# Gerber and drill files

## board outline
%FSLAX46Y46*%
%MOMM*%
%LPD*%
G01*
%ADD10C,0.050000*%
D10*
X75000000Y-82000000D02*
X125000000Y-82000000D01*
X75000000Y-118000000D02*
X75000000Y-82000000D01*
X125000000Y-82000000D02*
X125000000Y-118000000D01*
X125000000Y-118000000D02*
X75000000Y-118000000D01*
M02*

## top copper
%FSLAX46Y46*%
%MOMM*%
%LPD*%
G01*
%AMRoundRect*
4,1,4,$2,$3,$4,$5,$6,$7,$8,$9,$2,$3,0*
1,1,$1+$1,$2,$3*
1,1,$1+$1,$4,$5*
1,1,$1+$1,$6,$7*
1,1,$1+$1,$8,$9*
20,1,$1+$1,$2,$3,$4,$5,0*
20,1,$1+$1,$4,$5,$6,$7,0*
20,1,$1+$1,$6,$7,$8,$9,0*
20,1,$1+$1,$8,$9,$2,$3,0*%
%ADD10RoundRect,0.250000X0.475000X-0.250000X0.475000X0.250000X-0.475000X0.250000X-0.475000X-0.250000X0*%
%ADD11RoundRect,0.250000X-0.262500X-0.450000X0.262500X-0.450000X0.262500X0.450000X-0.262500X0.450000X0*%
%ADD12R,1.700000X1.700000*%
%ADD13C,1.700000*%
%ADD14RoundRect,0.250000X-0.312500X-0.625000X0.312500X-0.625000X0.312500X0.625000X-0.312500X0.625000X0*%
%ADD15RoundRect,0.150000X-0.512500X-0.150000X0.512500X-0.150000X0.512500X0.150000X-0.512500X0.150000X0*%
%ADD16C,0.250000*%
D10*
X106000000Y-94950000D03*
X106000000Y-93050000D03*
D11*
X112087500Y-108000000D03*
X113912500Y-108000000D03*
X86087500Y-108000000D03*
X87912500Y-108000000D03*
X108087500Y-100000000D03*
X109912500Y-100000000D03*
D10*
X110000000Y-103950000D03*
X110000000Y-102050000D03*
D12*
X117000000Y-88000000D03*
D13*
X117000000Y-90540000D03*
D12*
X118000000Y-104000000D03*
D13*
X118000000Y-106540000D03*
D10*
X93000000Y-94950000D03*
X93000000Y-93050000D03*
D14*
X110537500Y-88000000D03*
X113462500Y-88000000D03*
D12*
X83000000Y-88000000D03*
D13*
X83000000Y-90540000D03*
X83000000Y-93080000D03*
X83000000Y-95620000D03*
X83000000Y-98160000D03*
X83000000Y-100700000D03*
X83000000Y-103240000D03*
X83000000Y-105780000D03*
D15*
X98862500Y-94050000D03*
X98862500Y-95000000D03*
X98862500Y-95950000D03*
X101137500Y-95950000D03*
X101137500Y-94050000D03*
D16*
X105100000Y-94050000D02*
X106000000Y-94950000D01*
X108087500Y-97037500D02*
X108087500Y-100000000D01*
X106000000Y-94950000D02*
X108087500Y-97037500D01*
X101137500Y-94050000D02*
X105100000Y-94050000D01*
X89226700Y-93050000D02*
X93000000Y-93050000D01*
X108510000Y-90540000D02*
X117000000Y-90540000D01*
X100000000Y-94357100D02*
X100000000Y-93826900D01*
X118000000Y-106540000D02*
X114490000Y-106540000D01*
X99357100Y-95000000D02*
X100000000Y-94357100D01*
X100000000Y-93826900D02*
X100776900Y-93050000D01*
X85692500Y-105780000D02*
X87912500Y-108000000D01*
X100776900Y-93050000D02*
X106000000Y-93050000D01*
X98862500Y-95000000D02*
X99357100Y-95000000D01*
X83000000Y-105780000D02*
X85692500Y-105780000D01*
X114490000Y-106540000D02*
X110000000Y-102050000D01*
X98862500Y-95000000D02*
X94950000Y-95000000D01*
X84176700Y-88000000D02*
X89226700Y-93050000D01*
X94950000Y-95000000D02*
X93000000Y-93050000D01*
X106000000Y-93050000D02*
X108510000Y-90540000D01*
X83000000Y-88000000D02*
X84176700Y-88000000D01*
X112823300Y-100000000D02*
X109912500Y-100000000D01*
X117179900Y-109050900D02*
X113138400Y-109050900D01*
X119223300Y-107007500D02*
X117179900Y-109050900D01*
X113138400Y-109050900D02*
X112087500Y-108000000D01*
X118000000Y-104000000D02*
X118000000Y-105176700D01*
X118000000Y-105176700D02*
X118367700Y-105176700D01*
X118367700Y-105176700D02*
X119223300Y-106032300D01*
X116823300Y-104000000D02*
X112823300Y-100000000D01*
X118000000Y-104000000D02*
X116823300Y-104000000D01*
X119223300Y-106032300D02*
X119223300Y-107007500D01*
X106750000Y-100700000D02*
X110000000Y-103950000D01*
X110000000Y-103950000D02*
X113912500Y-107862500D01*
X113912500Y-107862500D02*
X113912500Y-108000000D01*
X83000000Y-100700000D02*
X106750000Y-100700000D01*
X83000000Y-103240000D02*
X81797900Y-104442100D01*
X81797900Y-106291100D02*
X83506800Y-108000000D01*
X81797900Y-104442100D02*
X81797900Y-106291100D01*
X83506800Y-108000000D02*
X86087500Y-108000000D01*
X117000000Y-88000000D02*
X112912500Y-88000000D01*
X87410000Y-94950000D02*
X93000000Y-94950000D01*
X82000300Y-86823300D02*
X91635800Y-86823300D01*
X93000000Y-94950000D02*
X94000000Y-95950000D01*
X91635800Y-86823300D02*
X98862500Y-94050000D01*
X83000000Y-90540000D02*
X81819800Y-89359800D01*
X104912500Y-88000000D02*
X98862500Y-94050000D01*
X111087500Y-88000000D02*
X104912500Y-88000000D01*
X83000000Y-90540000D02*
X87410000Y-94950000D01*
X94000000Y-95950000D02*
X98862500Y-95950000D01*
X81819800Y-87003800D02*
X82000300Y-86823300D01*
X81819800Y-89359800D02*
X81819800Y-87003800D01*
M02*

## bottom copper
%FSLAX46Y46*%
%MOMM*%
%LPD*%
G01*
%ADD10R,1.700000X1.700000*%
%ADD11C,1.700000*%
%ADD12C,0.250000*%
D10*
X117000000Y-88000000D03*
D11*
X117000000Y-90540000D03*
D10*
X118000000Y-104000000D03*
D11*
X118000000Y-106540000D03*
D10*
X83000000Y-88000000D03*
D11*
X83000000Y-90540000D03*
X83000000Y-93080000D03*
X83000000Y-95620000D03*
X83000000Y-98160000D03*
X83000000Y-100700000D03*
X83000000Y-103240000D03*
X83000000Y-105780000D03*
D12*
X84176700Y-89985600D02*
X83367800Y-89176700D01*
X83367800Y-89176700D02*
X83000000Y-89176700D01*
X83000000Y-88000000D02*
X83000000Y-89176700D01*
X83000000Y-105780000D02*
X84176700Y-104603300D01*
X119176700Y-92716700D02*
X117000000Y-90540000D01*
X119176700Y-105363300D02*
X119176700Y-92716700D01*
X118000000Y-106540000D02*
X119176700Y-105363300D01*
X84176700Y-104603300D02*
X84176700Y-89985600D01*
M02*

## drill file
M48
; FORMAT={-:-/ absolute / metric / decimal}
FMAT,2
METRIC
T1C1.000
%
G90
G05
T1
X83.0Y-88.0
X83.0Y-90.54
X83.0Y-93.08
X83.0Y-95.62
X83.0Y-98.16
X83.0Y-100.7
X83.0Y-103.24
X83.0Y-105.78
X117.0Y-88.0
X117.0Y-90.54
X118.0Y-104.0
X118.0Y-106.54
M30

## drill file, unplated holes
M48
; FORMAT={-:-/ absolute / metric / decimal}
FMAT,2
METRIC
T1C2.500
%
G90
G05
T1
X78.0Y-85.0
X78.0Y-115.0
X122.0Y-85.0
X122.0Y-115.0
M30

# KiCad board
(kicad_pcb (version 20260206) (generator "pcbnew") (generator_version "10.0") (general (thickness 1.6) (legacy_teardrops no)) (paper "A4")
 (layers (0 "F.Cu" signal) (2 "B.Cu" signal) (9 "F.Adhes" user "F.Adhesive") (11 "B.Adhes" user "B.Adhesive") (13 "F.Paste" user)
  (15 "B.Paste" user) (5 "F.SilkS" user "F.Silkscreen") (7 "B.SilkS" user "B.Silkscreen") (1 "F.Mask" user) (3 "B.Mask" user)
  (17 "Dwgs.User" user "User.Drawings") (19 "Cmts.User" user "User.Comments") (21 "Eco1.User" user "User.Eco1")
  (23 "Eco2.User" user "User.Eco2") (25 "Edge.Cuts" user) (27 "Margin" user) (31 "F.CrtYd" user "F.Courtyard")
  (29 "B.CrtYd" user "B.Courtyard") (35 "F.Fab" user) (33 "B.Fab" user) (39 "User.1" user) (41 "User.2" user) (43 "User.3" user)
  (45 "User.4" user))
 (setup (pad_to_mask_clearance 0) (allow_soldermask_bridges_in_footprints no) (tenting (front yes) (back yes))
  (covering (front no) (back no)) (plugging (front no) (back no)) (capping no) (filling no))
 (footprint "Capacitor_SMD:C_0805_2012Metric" (layer "F.Cu") (at 106 94 90)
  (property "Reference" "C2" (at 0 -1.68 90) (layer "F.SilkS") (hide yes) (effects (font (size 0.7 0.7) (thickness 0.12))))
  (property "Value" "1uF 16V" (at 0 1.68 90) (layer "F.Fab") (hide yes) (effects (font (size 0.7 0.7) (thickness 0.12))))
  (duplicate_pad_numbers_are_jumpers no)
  (pad "1" smd roundrect (at -0.95 0 90) (size 1 1.45) (layers "F.Cu" "F.Mask" "F.Paste") (roundrect_rratio 0.25) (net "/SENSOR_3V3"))
  (pad "2" smd roundrect (at 0.95 0 90) (size 1 1.45) (layers "F.Cu" "F.Mask" "F.Paste") (roundrect_rratio 0.25) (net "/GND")))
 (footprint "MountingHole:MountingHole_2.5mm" (layer "F.Cu") (at 78 85)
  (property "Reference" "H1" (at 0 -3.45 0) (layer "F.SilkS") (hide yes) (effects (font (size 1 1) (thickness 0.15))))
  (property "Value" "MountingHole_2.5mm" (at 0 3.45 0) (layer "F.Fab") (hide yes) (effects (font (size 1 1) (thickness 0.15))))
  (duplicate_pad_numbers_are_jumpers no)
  (pad "" np_thru_hole circle (at 0 0) (size 2.5 2.5) (drill 2.5) (layers "*.Cu" "*.Mask")))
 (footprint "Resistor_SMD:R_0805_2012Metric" (layer "F.Cu") (at 113 108)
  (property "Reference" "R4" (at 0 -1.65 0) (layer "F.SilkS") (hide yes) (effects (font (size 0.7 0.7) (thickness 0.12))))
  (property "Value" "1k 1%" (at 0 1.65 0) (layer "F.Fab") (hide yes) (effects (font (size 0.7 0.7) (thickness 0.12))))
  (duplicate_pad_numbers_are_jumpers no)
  (pad "1" smd roundrect (at -0.9125 0) (size 1.025 1.4) (layers "F.Cu" "F.Mask" "F.Paste") (roundrect_rratio 0.243902) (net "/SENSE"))
  (pad "2" smd roundrect (at 0.9125 0) (size 1.025 1.4) (layers "F.Cu" "F.Mask" "F.Paste") (roundrect_rratio 0.243902) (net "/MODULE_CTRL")))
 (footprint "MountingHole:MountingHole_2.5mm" (layer "F.Cu") (at 122 85)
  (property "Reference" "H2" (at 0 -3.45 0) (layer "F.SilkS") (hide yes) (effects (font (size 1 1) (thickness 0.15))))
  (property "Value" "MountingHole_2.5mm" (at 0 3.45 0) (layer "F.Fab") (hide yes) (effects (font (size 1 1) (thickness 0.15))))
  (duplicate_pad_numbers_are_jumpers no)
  (pad "" np_thru_hole circle (at 0 0) (size 2.5 2.5) (drill 2.5) (layers "*.Cu" "*.Mask")))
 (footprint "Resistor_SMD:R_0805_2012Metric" (layer "F.Cu") (at 87 108)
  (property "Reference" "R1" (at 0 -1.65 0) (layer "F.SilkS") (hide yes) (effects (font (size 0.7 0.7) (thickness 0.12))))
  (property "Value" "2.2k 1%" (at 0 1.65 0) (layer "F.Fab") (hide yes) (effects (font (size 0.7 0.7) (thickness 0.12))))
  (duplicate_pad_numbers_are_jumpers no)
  (pad "1" smd roundrect (at -0.9125 0) (size 1.025 1.4) (layers "F.Cu" "F.Mask" "F.Paste") (roundrect_rratio 0.243902) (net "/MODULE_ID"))
  (pad "2" smd roundrect (at 0.9125 0) (size 1.025 1.4) (layers "F.Cu" "F.Mask" "F.Paste") (roundrect_rratio 0.243902) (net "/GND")))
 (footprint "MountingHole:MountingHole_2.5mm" (layer "F.Cu") (at 78 115)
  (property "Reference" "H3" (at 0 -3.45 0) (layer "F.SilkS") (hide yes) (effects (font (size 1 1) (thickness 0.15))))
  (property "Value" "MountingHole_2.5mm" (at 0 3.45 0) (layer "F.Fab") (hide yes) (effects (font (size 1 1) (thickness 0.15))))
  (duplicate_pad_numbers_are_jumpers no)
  (pad "" np_thru_hole circle (at 0 0) (size 2.5 2.5) (drill 2.5) (layers "*.Cu" "*.Mask")))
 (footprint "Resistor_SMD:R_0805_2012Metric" (layer "F.Cu") (at 109 100)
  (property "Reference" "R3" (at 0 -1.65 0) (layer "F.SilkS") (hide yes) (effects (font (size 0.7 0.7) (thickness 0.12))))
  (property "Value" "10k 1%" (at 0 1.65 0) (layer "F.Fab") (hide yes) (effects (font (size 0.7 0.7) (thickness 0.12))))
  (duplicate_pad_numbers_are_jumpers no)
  (pad "1" smd roundrect (at -0.9125 0) (size 1.025 1.4) (layers "F.Cu" "F.Mask" "F.Paste") (roundrect_rratio 0.243902) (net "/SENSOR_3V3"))
  (pad "2" smd roundrect (at 0.9125 0) (size 1.025 1.4) (layers "F.Cu" "F.Mask" "F.Paste") (roundrect_rratio 0.243902) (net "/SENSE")))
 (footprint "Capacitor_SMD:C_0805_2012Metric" (layer "F.Cu") (at 110 103 90)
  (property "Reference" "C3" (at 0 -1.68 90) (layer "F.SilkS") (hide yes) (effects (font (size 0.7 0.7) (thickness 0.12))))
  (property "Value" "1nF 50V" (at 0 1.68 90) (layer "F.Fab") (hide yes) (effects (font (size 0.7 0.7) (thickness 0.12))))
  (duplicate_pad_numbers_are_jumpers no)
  (pad "1" smd roundrect (at -0.95 0 90) (size 1 1.45) (layers "F.Cu" "F.Mask" "F.Paste") (roundrect_rratio 0.25) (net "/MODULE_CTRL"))
  (pad "2" smd roundrect (at 0.95 0 90) (size 1 1.45) (layers "F.Cu" "F.Mask" "F.Paste") (roundrect_rratio 0.25) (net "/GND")))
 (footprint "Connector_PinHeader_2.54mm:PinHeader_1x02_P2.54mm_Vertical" (layer "F.Cu") (at 117 88)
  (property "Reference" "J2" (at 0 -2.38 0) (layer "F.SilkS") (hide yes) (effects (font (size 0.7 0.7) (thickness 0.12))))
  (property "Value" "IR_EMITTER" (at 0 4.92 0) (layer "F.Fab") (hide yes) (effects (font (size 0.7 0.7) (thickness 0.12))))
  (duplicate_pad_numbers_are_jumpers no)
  (pad "1" thru_hole rect (at 0 0) (size 1.7 1.7) (drill 1) (layers "*.Cu" "*.Mask") (remove_unused_layers no) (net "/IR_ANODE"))
  (pad "2" thru_hole circle (at 0 2.54) (size 1.7 1.7) (drill 1) (layers "*.Cu" "*.Mask") (remove_unused_layers no) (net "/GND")))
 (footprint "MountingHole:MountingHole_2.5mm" (layer "F.Cu") (at 122 115)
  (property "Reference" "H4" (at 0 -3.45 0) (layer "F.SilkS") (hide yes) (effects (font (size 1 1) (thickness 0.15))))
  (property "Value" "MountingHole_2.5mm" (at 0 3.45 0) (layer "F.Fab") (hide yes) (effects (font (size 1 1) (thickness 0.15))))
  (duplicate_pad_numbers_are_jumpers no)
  (pad "" np_thru_hole circle (at 0 0) (size 2.5 2.5) (drill 2.5) (layers "*.Cu" "*.Mask")))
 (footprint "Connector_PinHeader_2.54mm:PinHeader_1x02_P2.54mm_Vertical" (layer "F.Cu") (at 118 104)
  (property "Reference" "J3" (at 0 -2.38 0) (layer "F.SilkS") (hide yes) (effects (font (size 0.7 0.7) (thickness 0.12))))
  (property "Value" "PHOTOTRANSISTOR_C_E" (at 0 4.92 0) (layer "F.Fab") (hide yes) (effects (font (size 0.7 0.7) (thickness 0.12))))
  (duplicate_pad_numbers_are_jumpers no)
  (pad "1" thru_hole rect (at 0 0) (size 1.7 1.7) (drill 1) (layers "*.Cu" "*.Mask") (remove_unused_layers no) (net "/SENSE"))
  (pad "2" thru_hole circle (at 0 2.54) (size 1.7 1.7) (drill 1) (layers "*.Cu" "*.Mask") (remove_unused_layers no) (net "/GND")))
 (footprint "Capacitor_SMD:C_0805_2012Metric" (layer "F.Cu") (at 93 94 90)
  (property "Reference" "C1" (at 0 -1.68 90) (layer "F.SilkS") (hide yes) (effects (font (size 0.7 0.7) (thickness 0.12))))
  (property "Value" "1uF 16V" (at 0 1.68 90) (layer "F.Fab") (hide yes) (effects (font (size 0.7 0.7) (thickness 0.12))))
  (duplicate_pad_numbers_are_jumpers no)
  (pad "1" smd roundrect (at -0.95 0 90) (size 1 1.45) (layers "F.Cu" "F.Mask" "F.Paste") (roundrect_rratio 0.25) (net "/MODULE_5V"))
  (pad "2" smd roundrect (at 0.95 0 90) (size 1 1.45) (layers "F.Cu" "F.Mask" "F.Paste") (roundrect_rratio 0.25) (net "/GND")))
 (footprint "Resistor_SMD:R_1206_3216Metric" (layer "F.Cu") (at 112 88)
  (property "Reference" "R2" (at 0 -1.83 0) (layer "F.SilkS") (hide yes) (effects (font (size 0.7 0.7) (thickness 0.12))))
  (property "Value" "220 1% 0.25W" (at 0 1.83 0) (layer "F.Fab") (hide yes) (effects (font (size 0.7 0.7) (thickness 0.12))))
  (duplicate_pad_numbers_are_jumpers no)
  (pad "1" smd roundrect (at -1.4625 0) (size 1.125 1.75) (layers "F.Cu" "F.Mask" "F.Paste") (roundrect_rratio 0.222222) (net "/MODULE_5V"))
  (pad "2" smd roundrect (at 1.4625 0) (size 1.125 1.75) (layers "F.Cu" "F.Mask" "F.Paste") (roundrect_rratio 0.222222) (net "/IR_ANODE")))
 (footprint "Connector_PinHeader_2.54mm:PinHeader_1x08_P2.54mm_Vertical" (layer "F.Cu") (at 83 88)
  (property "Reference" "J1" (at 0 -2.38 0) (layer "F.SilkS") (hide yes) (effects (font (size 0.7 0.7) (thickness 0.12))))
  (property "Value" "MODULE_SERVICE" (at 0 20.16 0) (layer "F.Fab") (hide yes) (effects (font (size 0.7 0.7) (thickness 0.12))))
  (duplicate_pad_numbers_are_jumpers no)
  (pad "1" thru_hole rect (at 0 0) (size 1.7 1.7) (drill 1) (layers "*.Cu" "*.Mask") (remove_unused_layers no) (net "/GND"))
  (pad "2" thru_hole circle (at 0 2.54) (size 1.7 1.7) (drill 1) (layers "*.Cu" "*.Mask") (remove_unused_layers no) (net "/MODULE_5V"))
  (pad "3" thru_hole circle (at 0 5.08) (size 1.7 1.7) (drill 1) (layers "*.Cu" "*.Mask") (remove_unused_layers no)
   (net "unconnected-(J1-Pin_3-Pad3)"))
  (pad "4" thru_hole circle (at 0 7.62) (size 1.7 1.7) (drill 1) (layers "*.Cu" "*.Mask") (remove_unused_layers no)
   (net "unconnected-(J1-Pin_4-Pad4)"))
  (pad "5" thru_hole circle (at 0 10.16) (size 1.7 1.7) (drill 1) (layers "*.Cu" "*.Mask") (remove_unused_layers no)
   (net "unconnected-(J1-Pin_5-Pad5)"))
  (pad "6" thru_hole circle (at 0 12.7) (size 1.7 1.7) (drill 1) (layers "*.Cu" "*.Mask") (remove_unused_layers no) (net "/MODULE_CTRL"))
  (pad "7" thru_hole circle (at 0 15.24) (size 1.7 1.7) (drill 1) (layers "*.Cu" "*.Mask") (remove_unused_layers no) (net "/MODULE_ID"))
  (pad "8" thru_hole circle (at 0 17.78) (size 1.7 1.7) (drill 1) (layers "*.Cu" "*.Mask") (remove_unused_layers no) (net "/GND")))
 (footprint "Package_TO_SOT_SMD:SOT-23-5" (layer "F.Cu") (at 100 95)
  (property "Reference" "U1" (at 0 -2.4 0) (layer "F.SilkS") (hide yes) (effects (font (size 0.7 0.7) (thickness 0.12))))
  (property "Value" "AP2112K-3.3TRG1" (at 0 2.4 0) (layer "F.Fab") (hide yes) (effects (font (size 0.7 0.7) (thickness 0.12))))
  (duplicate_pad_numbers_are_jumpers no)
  (pad "1" smd roundrect (at -1.1375 -0.95) (size 1.325 0.6) (layers "F.Cu" "F.Mask" "F.Paste") (roundrect_rratio 0.25) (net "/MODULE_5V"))
  (pad "2" smd roundrect (at -1.1375 0) (size 1.325 0.6) (layers "F.Cu" "F.Mask" "F.Paste") (roundrect_rratio 0.25) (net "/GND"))
  (pad "3" smd roundrect (at -1.1375 0.95) (size 1.325 0.6) (layers "F.Cu" "F.Mask" "F.Paste") (roundrect_rratio 0.25) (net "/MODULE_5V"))
  (pad "4" smd roundrect (at 1.1375 0.95) (size 1.325 0.6) (layers "F.Cu" "F.Mask" "F.Paste") (roundrect_rratio 0.25)
   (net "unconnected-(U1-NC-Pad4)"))
  (pad "5" smd roundrect (at 1.1375 -0.95) (size 1.325 0.6) (layers "F.Cu" "F.Mask" "F.Paste") (roundrect_rratio 0.25) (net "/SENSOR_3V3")))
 (gr_line (start 75 82) (end 125 82) (stroke (width 0.05) (type default)) (layer "Edge.Cuts"))
 (gr_line (start 75 118) (end 75 82) (stroke (width 0.05) (type default)) (layer "Edge.Cuts"))
 (gr_line (start 125 82) (end 125 118) (stroke (width 0.05) (type default)) (layer "Edge.Cuts"))
 (gr_line (start 125 118) (end 75 118) (stroke (width 0.05) (type default)) (layer "Edge.Cuts"))
 (segment (start 105.1 94.05) (end 106 94.95) (width 0.25) (layer "F.Cu") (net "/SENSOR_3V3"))
 (segment (start 108.0875 97.0375) (end 108.0875 100) (width 0.25) (layer "F.Cu") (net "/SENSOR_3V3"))
 (segment (start 106 94.95) (end 108.0875 97.0375) (width 0.25) (layer "F.Cu") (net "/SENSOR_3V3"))
 (segment (start 101.1375 94.05) (end 105.1 94.05) (width 0.25) (layer "F.Cu") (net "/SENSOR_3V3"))
 (segment (start 89.2267 93.05) (end 93 93.05) (width 0.25) (layer "F.Cu") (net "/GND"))
 (segment (start 108.51 90.54) (end 117 90.54) (width 0.25) (layer "F.Cu") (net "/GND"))
 (segment (start 100 94.3571) (end 100 93.8269) (width 0.25) (layer "F.Cu") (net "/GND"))
 (segment (start 118 106.54) (end 114.49 106.54) (width 0.25) (layer "F.Cu") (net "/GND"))
 (segment (start 99.3571 95) (end 100 94.3571) (width 0.25) (layer "F.Cu") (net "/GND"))
 (segment (start 100 93.8269) (end 100.7769 93.05) (width 0.25) (layer "F.Cu") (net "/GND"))
 (segment (start 85.6925 105.78) (end 87.9125 108) (width 0.25) (layer "F.Cu") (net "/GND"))
 (segment (start 100.7769 93.05) (end 106 93.05) (width 0.25) (layer "F.Cu") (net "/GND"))
 (segment (start 98.8625 95) (end 99.3571 95) (width 0.25) (layer "F.Cu") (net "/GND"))
 (segment (start 83 105.78) (end 85.6925 105.78) (width 0.25) (layer "F.Cu") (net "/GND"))
 (segment (start 114.49 106.54) (end 110 102.05) (width 0.25) (layer "F.Cu") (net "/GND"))
 (segment (start 98.8625 95) (end 94.95 95) (width 0.25) (layer "F.Cu") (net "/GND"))
 (segment (start 84.1767 88) (end 89.2267 93.05) (width 0.25) (layer "F.Cu") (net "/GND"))
 (segment (start 94.95 95) (end 93 93.05) (width 0.25) (layer "F.Cu") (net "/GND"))
 (segment (start 106 93.05) (end 108.51 90.54) (width 0.25) (layer "F.Cu") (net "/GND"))
 (segment (start 83 88) (end 84.1767 88) (width 0.25) (layer "F.Cu") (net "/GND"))
 (segment (start 84.1767 89.9856) (end 83.3678 89.1767) (width 0.25) (layer "B.Cu") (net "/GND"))
 (segment (start 83.3678 89.1767) (end 83 89.1767) (width 0.25) (layer "B.Cu") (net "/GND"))
 (segment (start 83 88) (end 83 89.1767) (width 0.25) (layer "B.Cu") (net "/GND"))
 (segment (start 83 105.78) (end 84.1767 104.6033) (width 0.25) (layer "B.Cu") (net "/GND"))
 (segment (start 119.1767 92.7167) (end 117 90.54) (width 0.25) (layer "B.Cu") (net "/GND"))
 (segment (start 119.1767 105.3633) (end 119.1767 92.7167) (width 0.25) (layer "B.Cu") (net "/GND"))
 (segment (start 118 106.54) (end 119.1767 105.3633) (width 0.25) (layer "B.Cu") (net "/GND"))
 (segment (start 84.1767 104.6033) (end 84.1767 89.9856) (width 0.25) (layer "B.Cu") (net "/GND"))
 (segment (start 112.8233 100) (end 109.9125 100) (width 0.25) (layer "F.Cu") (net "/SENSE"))
 (segment (start 117.1799 109.0509) (end 113.1384 109.0509) (width 0.25) (layer "F.Cu") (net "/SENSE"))
 (segment (start 119.2233 107.0075) (end 117.1799 109.0509) (width 0.25) (layer "F.Cu") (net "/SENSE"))
 (segment (start 113.1384 109.0509) (end 112.0875 108) (width 0.25) (layer "F.Cu") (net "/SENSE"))
 (segment (start 118 104) (end 118 105.1767) (width 0.25) (layer "F.Cu") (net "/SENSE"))
 (segment (start 118 105.1767) (end 118.3677 105.1767) (width 0.25) (layer "F.Cu") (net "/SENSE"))
 (segment (start 118.3677 105.1767) (end 119.2233 106.0323) (width 0.25) (layer "F.Cu") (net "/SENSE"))
 (segment (start 116.8233 104) (end 112.8233 100) (width 0.25) (layer "F.Cu") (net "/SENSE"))
 (segment (start 118 104) (end 116.8233 104) (width 0.25) (layer "F.Cu") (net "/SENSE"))
 (segment (start 119.2233 106.0323) (end 119.2233 107.0075) (width 0.25) (layer "F.Cu") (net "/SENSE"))
 (segment (start 106.75 100.7) (end 110 103.95) (width 0.25) (layer "F.Cu") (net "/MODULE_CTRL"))
 (segment (start 110 103.95) (end 113.9125 107.8625) (width 0.25) (layer "F.Cu") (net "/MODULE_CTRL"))
 (segment (start 113.9125 107.8625) (end 113.9125 108) (width 0.25) (layer "F.Cu") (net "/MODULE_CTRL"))
 (segment (start 83 100.7) (end 106.75 100.7) (width 0.25) (layer "F.Cu") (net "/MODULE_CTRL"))
 (segment (start 83 103.24) (end 81.7979 104.4421) (width 0.25) (layer "F.Cu") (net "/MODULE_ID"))
 (segment (start 81.7979 106.2911) (end 83.5068 108) (width 0.25) (layer "F.Cu") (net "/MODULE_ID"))
 (segment (start 81.7979 104.4421) (end 81.7979 106.2911) (width 0.25) (layer "F.Cu") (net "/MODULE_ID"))
 (segment (start 83.5068 108) (end 86.0875 108) (width 0.25) (layer "F.Cu") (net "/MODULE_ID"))
 (segment (start 117 88) (end 112.9125 88) (width 0.25) (layer "F.Cu") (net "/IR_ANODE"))
 (segment (start 87.41 94.95) (end 93 94.95) (width 0.25) (layer "F.Cu") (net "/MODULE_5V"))
 (segment (start 82.0003 86.8233) (end 91.6358 86.8233) (width 0.25) (layer "F.Cu") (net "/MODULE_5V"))
 (segment (start 93 94.95) (end 94 95.95) (width 0.25) (layer "F.Cu") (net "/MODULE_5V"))
 (segment (start 91.6358 86.8233) (end 98.8625 94.05) (width 0.25) (layer "F.Cu") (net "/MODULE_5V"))
 (segment (start 83 90.54) (end 81.8198 89.3598) (width 0.25) (layer "F.Cu") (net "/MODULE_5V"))
 (segment (start 104.9125 88) (end 98.8625 94.05) (width 0.25) (layer "F.Cu") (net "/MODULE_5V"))
 (segment (start 111.0875 88) (end 104.9125 88) (width 0.25) (layer "F.Cu") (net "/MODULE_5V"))
 (segment (start 83 90.54) (end 87.41 94.95) (width 0.25) (layer "F.Cu") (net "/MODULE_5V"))
 (segment (start 94 95.95) (end 98.8625 95.95) (width 0.25) (layer "F.Cu") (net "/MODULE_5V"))
 (segment (start 81.8198 87.0038) (end 82.0003 86.8233) (width 0.25) (layer "F.Cu") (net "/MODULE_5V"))
 (segment (start 81.8198 89.3598) (end 81.8198 87.0038) (width 0.25) (layer "F.Cu") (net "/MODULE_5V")))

